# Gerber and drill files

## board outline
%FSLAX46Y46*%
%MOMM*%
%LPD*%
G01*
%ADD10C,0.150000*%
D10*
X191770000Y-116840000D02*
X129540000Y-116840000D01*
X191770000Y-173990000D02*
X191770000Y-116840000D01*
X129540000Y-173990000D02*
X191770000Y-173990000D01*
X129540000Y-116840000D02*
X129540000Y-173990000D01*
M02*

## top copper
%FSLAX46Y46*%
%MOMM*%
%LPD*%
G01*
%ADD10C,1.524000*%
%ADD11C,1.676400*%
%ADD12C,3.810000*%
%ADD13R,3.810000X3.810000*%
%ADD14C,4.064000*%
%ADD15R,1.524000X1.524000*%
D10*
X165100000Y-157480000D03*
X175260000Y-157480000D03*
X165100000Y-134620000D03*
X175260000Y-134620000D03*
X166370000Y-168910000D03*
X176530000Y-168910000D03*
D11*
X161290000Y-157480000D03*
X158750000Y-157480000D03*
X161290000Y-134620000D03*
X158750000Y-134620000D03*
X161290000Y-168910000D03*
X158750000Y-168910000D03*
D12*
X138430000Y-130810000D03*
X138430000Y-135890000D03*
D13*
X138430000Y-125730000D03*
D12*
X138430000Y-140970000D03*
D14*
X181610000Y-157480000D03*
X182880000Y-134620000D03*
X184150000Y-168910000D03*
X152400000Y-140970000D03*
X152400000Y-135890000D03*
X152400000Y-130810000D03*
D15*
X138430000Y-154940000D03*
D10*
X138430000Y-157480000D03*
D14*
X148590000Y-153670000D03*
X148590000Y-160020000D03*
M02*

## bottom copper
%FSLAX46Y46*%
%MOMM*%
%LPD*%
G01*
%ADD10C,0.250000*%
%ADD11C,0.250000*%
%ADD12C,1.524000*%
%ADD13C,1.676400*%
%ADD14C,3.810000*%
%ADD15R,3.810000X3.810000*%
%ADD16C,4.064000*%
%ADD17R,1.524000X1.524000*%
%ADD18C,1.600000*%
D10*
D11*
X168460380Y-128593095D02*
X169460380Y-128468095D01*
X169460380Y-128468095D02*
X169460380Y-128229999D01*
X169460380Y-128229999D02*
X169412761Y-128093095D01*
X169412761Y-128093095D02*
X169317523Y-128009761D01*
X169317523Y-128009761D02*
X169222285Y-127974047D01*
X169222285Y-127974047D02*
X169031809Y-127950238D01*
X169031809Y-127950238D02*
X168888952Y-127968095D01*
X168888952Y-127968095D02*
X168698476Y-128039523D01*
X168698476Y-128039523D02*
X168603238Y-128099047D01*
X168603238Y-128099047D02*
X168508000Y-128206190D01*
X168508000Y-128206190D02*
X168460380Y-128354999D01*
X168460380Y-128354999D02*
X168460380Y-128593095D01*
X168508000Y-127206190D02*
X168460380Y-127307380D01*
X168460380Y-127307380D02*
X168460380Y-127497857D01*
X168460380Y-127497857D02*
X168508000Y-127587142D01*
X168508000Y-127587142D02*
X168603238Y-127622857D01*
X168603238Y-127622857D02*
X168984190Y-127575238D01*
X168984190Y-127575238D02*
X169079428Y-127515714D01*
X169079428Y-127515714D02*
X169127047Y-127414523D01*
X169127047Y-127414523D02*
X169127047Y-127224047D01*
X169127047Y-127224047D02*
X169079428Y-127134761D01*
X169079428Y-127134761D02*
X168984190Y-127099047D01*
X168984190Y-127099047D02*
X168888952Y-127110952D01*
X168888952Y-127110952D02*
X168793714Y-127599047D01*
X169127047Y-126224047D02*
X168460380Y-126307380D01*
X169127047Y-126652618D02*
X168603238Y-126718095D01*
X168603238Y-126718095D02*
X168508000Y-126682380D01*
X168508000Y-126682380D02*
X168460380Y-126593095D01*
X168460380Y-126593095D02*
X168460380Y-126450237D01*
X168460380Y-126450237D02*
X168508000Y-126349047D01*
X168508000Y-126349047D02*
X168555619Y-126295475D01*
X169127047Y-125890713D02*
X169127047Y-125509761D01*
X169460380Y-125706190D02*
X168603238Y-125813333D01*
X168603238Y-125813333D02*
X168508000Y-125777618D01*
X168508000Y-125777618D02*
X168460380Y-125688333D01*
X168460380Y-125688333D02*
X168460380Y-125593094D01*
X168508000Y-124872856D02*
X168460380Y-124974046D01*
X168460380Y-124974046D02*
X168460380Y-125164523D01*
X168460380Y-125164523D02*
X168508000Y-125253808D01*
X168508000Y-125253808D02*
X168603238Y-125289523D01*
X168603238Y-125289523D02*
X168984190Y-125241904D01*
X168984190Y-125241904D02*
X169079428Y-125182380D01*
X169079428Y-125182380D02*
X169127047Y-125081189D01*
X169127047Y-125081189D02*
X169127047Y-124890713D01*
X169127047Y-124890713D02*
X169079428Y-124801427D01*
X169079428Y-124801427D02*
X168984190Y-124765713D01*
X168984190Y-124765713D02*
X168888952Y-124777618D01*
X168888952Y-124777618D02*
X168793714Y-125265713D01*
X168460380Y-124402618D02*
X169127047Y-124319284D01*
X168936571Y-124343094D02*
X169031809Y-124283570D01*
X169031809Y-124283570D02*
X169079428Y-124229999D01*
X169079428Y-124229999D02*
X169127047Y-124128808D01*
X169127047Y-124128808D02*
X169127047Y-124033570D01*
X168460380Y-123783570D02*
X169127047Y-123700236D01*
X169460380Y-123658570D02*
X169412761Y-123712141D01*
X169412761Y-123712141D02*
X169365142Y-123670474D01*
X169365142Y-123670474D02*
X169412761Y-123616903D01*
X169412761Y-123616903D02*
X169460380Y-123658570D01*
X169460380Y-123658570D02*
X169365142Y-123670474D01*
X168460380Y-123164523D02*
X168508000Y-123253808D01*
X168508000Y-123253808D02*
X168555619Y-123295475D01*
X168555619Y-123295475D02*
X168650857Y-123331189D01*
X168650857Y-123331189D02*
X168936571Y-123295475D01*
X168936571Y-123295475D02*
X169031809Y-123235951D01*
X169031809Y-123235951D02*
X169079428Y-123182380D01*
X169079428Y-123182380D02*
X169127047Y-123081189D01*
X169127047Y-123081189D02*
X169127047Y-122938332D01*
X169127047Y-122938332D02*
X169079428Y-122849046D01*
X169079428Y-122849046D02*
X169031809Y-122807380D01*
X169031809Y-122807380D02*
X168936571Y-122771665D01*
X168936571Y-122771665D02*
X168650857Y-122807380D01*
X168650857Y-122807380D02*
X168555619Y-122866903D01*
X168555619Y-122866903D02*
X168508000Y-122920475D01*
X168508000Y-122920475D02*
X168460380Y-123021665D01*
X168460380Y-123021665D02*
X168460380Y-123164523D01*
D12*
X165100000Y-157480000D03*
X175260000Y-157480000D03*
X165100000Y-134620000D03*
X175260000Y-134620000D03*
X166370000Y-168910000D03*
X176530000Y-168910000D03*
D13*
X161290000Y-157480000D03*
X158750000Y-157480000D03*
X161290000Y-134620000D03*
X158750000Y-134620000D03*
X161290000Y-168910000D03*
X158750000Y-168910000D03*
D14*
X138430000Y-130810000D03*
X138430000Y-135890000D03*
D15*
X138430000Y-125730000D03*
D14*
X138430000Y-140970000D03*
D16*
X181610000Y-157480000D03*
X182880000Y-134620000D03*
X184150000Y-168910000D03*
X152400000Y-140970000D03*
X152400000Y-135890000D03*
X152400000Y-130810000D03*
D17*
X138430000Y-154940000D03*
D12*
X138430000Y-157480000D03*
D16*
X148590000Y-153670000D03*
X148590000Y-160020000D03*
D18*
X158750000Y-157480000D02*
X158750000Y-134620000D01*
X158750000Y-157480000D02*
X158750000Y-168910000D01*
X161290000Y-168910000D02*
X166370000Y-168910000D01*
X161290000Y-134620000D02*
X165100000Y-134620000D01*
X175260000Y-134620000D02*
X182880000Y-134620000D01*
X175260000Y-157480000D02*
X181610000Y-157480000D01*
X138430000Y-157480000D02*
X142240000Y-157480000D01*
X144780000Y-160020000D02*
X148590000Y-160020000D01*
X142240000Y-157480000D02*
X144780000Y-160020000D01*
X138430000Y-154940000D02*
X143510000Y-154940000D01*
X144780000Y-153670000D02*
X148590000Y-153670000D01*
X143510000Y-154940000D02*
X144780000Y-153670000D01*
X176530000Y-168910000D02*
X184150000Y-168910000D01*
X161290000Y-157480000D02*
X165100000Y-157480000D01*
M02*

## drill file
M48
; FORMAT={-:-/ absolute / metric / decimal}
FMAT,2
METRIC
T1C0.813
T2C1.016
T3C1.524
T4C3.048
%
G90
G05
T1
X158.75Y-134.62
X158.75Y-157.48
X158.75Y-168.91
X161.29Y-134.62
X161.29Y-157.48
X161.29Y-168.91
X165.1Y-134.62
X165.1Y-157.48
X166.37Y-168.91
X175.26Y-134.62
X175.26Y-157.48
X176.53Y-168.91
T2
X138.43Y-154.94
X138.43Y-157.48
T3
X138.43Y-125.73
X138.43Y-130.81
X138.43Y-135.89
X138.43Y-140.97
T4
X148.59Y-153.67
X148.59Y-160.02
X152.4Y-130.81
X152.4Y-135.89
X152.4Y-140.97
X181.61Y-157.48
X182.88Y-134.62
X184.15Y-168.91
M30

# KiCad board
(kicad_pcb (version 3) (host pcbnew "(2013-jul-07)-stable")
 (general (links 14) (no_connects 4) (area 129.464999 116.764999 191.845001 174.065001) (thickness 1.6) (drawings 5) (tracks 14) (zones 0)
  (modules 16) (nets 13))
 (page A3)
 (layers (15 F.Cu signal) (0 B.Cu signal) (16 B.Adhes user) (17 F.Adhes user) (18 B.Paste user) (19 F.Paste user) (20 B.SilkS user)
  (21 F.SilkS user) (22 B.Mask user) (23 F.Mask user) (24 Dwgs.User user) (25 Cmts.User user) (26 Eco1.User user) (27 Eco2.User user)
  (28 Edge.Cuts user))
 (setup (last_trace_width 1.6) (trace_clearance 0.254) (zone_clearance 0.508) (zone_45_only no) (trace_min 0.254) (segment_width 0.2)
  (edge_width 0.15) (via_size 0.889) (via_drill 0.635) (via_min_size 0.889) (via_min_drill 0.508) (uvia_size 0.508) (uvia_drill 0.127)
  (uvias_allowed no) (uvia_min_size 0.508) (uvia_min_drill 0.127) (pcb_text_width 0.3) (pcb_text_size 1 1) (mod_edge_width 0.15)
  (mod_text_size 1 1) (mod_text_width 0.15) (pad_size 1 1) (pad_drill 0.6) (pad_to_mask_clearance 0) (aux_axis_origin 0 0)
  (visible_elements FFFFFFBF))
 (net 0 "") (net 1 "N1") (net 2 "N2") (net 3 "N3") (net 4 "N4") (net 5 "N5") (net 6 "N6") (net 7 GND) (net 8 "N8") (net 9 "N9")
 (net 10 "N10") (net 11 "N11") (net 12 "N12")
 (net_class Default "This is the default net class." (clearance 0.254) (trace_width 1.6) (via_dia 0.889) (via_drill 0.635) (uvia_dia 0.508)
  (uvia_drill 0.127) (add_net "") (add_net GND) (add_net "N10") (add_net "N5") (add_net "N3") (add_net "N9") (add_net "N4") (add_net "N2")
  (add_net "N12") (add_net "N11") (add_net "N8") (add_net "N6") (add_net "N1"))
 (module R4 (layer F.Cu) (at 170.18 157.48) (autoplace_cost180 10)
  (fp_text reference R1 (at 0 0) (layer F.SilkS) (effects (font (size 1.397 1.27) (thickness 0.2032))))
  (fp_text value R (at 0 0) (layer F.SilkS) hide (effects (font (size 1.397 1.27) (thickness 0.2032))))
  (pad 1 thru_hole circle (at -5.08 0) (size 1.524 1.524) (drill 0.8128) (layers *.Cu *.Mask F.SilkS) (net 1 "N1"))
  (pad 2 thru_hole circle (at 5.08 0) (size 1.524 1.524) (drill 0.8128) (layers *.Cu *.Mask F.SilkS) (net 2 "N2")))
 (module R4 (layer F.Cu) (at 170.18 134.62) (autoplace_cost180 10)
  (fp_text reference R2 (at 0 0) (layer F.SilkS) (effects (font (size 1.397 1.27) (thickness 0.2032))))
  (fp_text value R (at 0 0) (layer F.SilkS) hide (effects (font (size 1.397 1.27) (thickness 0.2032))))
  (pad 1 thru_hole circle (at -5.08 0) (size 1.524 1.524) (drill 0.8128) (layers *.Cu *.Mask F.SilkS) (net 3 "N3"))
  (pad 2 thru_hole circle (at 5.08 0) (size 1.524 1.524) (drill 0.8128) (layers *.Cu *.Mask F.SilkS) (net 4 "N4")))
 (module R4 (layer F.Cu) (at 171.45 168.91) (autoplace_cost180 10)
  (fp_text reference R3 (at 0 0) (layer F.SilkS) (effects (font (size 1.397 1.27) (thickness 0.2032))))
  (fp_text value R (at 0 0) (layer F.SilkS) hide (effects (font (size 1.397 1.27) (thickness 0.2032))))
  (pad 1 thru_hole circle (at -5.08 0) (size 1.524 1.524) (drill 0.8128) (layers *.Cu *.Mask F.SilkS) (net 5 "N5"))
  (pad 2 thru_hole circle (at 5.08 0) (size 1.524 1.524) (drill 0.8128) (layers *.Cu *.Mask F.SilkS) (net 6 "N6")))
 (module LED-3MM (layer F.Cu) (at 160.02 157.48 180)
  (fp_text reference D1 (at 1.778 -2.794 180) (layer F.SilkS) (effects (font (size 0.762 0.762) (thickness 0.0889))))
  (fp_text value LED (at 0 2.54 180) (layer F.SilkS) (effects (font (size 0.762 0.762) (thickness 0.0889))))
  (pad 1 thru_hole circle (at -1.27 0 180) (size 1.6764 1.6764) (drill 0.8128) (layers *.Cu *.Mask F.SilkS) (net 1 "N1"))
  (pad 2 thru_hole circle (at 1.27 0 180) (size 1.6764 1.6764) (drill 0.8128) (layers *.Cu *.Mask F.SilkS) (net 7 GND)))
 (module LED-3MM (layer F.Cu) (at 160.02 134.62 180)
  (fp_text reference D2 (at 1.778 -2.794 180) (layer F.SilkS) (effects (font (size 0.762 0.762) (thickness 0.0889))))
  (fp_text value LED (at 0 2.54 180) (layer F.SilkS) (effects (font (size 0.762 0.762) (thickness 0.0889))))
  (pad 1 thru_hole circle (at -1.27 0 180) (size 1.6764 1.6764) (drill 0.8128) (layers *.Cu *.Mask F.SilkS) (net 3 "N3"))
  (pad 2 thru_hole circle (at 1.27 0 180) (size 1.6764 1.6764) (drill 0.8128) (layers *.Cu *.Mask F.SilkS) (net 7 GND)))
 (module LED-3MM (layer F.Cu) (at 160.02 168.91 180)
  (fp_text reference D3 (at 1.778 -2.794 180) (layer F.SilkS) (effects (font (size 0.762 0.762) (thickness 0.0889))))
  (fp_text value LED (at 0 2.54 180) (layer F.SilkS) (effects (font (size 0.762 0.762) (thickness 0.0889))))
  (pad 1 thru_hole circle (at -1.27 0 180) (size 1.6764 1.6764) (drill 0.8128) (layers *.Cu *.Mask F.SilkS) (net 5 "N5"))
  (pad 2 thru_hole circle (at 1.27 0 180) (size 1.6764 1.6764) (drill 0.8128) (layers *.Cu *.Mask F.SilkS) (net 7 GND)))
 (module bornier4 (layer F.Cu) (at 138.43 133.35 270)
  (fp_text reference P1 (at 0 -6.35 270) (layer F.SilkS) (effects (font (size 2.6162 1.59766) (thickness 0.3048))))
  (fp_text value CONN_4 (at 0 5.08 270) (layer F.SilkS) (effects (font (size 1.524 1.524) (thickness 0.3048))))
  (pad 2 thru_hole circle (at -2.54 0 270) (size 3.81 3.81) (drill 1.524) (layers *.Cu *.Mask F.SilkS) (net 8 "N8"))
  (pad 3 thru_hole circle (at 2.54 0 270) (size 3.81 3.81) (drill 1.524) (layers *.Cu *.Mask F.SilkS) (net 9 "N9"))
  (pad 1 thru_hole rect (at -7.62 0 270) (size 3.81 3.81) (drill 1.524) (layers *.Cu *.Mask F.SilkS) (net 7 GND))
  (pad 4 thru_hole circle (at 7.62 0 270) (size 3.81 3.81) (drill 1.524) (layers *.Cu *.Mask F.SilkS) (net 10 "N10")))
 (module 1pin (layer F.Cu) (at 181.61 157.48)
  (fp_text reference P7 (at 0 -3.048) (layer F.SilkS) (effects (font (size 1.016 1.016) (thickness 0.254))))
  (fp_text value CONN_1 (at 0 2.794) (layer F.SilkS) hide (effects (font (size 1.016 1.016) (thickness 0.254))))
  (pad 1 thru_hole circle (at 0 0) (size 4.064 4.064) (drill 3.048) (layers *.Cu *.Mask F.SilkS) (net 2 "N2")))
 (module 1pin (layer F.Cu) (at 182.88 134.62)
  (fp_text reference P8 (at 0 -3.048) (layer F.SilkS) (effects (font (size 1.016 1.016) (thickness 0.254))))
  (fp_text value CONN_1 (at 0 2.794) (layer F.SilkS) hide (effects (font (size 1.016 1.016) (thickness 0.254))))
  (pad 1 thru_hole circle (at 0 0) (size 4.064 4.064) (drill 3.048) (layers *.Cu *.Mask F.SilkS) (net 4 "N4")))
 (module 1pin (layer F.Cu) (at 184.15 168.91)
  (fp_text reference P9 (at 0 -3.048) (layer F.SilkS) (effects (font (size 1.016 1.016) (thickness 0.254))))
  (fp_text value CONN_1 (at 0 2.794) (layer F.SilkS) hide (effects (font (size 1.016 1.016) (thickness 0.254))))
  (pad 1 thru_hole circle (at 0 0) (size 4.064 4.064) (drill 3.048) (layers *.Cu *.Mask F.SilkS) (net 6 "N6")))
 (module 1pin (layer F.Cu) (at 152.4 140.97)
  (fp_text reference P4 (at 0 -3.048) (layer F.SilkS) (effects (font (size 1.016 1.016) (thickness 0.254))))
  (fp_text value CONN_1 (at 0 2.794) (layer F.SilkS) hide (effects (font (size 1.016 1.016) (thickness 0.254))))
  (pad 1 thru_hole circle (at 0 0) (size 4.064 4.064) (drill 3.048) (layers *.Cu *.Mask F.SilkS) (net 10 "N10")))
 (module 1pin (layer F.Cu) (at 152.4 135.89)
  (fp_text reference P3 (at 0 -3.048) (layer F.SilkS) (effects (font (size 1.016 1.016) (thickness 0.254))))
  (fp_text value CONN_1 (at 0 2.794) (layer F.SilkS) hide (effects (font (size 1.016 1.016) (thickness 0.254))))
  (pad 1 thru_hole circle (at 0 0) (size 4.064 4.064) (drill 3.048) (layers *.Cu *.Mask F.SilkS) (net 9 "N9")))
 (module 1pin (layer F.Cu) (at 152.4 130.81)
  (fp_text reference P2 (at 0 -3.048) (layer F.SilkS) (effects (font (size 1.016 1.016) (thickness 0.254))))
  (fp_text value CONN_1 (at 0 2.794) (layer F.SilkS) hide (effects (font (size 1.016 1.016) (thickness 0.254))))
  (pad 1 thru_hole circle (at 0 0) (size 4.064 4.064) (drill 3.048) (layers *.Cu *.Mask F.SilkS) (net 8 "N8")))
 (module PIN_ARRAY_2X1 (layer F.Cu) (at 138.43 156.21 270)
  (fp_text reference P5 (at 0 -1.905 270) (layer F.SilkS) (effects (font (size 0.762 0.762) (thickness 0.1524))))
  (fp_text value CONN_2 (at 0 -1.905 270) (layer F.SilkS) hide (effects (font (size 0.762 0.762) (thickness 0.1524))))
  (pad 1 thru_hole rect (at -1.27 0 270) (size 1.524 1.524) (drill 1.016) (layers *.Cu *.Mask F.SilkS) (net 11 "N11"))
  (pad 2 thru_hole circle (at 1.27 0 270) (size 1.524 1.524) (drill 1.016) (layers *.Cu *.Mask F.SilkS) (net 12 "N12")))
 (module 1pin (layer F.Cu) (at 148.59 153.67)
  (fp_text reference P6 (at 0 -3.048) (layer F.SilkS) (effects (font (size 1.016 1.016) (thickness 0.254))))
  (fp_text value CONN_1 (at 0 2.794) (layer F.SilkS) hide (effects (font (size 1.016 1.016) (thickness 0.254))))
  (pad 1 thru_hole circle (at 0 0) (size 4.064 4.064) (drill 3.048) (layers *.Cu *.Mask F.SilkS) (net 11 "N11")))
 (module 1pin (layer F.Cu) (at 148.59 160.02)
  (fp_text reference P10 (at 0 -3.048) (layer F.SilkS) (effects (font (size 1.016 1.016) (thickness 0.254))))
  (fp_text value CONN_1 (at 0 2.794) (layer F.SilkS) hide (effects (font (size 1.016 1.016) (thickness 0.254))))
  (pad 1 thru_hole circle (at 0 0) (size 4.064 4.064) (drill 3.048) (layers *.Cu *.Mask F.SilkS) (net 12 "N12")))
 (gr_line (start 191.77 116.84) (end 129.54 116.84) (angle 90) (layer Edge.Cuts) (width 0.15))
 (gr_line (start 191.77 173.99) (end 191.77 116.84) (angle 90) (layer Edge.Cuts) (width 0.15))
 (gr_line (start 129.54 173.99) (end 191.77 173.99) (angle 90) (layer Edge.Cuts) (width 0.15))
 (gr_line (start 129.54 116.84) (end 129.54 173.99) (angle 90) (layer Edge.Cuts) (width 0.15))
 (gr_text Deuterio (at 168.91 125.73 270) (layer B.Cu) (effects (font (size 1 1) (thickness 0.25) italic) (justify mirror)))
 (segment (start 158.75 157.48) (end 158.75 134.62) (width 1.6) (layer B.Cu) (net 7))
 (segment (start 158.75 157.48) (end 158.75 168.91) (width 1.6) (layer B.Cu) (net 7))
 (segment (start 161.29 168.91) (end 166.37 168.91) (width 1.6) (layer B.Cu) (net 5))
 (segment (start 161.29 134.62) (end 165.1 134.62) (width 1.6) (layer B.Cu) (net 3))
 (segment (start 175.26 134.62) (end 182.88 134.62) (width 1.6) (layer B.Cu) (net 4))
 (segment (start 175.26 157.48) (end 181.61 157.48) (width 1.6) (layer B.Cu) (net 2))
 (segment (start 138.43 157.48) (end 142.24 157.48) (width 1.6) (layer B.Cu) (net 12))
 (segment (start 144.78 160.02) (end 148.59 160.02) (width 1.6) (layer B.Cu) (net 12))
 (segment (start 142.24 157.48) (end 144.78 160.02) (width 1.6) (layer B.Cu) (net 12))
 (segment (start 138.43 154.94) (end 143.51 154.94) (width 1.6) (layer B.Cu) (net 11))
 (segment (start 144.78 153.67) (end 148.59 153.67) (width 1.6) (layer B.Cu) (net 11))
 (segment (start 143.51 154.94) (end 144.78 153.67) (width 1.6) (layer B.Cu) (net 11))
 (segment (start 176.53 168.91) (end 184.15 168.91) (width 1.6) (layer B.Cu) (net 6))
 (segment (start 161.29 157.48) (end 165.1 157.48) (width 1.6) (layer B.Cu) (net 1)))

